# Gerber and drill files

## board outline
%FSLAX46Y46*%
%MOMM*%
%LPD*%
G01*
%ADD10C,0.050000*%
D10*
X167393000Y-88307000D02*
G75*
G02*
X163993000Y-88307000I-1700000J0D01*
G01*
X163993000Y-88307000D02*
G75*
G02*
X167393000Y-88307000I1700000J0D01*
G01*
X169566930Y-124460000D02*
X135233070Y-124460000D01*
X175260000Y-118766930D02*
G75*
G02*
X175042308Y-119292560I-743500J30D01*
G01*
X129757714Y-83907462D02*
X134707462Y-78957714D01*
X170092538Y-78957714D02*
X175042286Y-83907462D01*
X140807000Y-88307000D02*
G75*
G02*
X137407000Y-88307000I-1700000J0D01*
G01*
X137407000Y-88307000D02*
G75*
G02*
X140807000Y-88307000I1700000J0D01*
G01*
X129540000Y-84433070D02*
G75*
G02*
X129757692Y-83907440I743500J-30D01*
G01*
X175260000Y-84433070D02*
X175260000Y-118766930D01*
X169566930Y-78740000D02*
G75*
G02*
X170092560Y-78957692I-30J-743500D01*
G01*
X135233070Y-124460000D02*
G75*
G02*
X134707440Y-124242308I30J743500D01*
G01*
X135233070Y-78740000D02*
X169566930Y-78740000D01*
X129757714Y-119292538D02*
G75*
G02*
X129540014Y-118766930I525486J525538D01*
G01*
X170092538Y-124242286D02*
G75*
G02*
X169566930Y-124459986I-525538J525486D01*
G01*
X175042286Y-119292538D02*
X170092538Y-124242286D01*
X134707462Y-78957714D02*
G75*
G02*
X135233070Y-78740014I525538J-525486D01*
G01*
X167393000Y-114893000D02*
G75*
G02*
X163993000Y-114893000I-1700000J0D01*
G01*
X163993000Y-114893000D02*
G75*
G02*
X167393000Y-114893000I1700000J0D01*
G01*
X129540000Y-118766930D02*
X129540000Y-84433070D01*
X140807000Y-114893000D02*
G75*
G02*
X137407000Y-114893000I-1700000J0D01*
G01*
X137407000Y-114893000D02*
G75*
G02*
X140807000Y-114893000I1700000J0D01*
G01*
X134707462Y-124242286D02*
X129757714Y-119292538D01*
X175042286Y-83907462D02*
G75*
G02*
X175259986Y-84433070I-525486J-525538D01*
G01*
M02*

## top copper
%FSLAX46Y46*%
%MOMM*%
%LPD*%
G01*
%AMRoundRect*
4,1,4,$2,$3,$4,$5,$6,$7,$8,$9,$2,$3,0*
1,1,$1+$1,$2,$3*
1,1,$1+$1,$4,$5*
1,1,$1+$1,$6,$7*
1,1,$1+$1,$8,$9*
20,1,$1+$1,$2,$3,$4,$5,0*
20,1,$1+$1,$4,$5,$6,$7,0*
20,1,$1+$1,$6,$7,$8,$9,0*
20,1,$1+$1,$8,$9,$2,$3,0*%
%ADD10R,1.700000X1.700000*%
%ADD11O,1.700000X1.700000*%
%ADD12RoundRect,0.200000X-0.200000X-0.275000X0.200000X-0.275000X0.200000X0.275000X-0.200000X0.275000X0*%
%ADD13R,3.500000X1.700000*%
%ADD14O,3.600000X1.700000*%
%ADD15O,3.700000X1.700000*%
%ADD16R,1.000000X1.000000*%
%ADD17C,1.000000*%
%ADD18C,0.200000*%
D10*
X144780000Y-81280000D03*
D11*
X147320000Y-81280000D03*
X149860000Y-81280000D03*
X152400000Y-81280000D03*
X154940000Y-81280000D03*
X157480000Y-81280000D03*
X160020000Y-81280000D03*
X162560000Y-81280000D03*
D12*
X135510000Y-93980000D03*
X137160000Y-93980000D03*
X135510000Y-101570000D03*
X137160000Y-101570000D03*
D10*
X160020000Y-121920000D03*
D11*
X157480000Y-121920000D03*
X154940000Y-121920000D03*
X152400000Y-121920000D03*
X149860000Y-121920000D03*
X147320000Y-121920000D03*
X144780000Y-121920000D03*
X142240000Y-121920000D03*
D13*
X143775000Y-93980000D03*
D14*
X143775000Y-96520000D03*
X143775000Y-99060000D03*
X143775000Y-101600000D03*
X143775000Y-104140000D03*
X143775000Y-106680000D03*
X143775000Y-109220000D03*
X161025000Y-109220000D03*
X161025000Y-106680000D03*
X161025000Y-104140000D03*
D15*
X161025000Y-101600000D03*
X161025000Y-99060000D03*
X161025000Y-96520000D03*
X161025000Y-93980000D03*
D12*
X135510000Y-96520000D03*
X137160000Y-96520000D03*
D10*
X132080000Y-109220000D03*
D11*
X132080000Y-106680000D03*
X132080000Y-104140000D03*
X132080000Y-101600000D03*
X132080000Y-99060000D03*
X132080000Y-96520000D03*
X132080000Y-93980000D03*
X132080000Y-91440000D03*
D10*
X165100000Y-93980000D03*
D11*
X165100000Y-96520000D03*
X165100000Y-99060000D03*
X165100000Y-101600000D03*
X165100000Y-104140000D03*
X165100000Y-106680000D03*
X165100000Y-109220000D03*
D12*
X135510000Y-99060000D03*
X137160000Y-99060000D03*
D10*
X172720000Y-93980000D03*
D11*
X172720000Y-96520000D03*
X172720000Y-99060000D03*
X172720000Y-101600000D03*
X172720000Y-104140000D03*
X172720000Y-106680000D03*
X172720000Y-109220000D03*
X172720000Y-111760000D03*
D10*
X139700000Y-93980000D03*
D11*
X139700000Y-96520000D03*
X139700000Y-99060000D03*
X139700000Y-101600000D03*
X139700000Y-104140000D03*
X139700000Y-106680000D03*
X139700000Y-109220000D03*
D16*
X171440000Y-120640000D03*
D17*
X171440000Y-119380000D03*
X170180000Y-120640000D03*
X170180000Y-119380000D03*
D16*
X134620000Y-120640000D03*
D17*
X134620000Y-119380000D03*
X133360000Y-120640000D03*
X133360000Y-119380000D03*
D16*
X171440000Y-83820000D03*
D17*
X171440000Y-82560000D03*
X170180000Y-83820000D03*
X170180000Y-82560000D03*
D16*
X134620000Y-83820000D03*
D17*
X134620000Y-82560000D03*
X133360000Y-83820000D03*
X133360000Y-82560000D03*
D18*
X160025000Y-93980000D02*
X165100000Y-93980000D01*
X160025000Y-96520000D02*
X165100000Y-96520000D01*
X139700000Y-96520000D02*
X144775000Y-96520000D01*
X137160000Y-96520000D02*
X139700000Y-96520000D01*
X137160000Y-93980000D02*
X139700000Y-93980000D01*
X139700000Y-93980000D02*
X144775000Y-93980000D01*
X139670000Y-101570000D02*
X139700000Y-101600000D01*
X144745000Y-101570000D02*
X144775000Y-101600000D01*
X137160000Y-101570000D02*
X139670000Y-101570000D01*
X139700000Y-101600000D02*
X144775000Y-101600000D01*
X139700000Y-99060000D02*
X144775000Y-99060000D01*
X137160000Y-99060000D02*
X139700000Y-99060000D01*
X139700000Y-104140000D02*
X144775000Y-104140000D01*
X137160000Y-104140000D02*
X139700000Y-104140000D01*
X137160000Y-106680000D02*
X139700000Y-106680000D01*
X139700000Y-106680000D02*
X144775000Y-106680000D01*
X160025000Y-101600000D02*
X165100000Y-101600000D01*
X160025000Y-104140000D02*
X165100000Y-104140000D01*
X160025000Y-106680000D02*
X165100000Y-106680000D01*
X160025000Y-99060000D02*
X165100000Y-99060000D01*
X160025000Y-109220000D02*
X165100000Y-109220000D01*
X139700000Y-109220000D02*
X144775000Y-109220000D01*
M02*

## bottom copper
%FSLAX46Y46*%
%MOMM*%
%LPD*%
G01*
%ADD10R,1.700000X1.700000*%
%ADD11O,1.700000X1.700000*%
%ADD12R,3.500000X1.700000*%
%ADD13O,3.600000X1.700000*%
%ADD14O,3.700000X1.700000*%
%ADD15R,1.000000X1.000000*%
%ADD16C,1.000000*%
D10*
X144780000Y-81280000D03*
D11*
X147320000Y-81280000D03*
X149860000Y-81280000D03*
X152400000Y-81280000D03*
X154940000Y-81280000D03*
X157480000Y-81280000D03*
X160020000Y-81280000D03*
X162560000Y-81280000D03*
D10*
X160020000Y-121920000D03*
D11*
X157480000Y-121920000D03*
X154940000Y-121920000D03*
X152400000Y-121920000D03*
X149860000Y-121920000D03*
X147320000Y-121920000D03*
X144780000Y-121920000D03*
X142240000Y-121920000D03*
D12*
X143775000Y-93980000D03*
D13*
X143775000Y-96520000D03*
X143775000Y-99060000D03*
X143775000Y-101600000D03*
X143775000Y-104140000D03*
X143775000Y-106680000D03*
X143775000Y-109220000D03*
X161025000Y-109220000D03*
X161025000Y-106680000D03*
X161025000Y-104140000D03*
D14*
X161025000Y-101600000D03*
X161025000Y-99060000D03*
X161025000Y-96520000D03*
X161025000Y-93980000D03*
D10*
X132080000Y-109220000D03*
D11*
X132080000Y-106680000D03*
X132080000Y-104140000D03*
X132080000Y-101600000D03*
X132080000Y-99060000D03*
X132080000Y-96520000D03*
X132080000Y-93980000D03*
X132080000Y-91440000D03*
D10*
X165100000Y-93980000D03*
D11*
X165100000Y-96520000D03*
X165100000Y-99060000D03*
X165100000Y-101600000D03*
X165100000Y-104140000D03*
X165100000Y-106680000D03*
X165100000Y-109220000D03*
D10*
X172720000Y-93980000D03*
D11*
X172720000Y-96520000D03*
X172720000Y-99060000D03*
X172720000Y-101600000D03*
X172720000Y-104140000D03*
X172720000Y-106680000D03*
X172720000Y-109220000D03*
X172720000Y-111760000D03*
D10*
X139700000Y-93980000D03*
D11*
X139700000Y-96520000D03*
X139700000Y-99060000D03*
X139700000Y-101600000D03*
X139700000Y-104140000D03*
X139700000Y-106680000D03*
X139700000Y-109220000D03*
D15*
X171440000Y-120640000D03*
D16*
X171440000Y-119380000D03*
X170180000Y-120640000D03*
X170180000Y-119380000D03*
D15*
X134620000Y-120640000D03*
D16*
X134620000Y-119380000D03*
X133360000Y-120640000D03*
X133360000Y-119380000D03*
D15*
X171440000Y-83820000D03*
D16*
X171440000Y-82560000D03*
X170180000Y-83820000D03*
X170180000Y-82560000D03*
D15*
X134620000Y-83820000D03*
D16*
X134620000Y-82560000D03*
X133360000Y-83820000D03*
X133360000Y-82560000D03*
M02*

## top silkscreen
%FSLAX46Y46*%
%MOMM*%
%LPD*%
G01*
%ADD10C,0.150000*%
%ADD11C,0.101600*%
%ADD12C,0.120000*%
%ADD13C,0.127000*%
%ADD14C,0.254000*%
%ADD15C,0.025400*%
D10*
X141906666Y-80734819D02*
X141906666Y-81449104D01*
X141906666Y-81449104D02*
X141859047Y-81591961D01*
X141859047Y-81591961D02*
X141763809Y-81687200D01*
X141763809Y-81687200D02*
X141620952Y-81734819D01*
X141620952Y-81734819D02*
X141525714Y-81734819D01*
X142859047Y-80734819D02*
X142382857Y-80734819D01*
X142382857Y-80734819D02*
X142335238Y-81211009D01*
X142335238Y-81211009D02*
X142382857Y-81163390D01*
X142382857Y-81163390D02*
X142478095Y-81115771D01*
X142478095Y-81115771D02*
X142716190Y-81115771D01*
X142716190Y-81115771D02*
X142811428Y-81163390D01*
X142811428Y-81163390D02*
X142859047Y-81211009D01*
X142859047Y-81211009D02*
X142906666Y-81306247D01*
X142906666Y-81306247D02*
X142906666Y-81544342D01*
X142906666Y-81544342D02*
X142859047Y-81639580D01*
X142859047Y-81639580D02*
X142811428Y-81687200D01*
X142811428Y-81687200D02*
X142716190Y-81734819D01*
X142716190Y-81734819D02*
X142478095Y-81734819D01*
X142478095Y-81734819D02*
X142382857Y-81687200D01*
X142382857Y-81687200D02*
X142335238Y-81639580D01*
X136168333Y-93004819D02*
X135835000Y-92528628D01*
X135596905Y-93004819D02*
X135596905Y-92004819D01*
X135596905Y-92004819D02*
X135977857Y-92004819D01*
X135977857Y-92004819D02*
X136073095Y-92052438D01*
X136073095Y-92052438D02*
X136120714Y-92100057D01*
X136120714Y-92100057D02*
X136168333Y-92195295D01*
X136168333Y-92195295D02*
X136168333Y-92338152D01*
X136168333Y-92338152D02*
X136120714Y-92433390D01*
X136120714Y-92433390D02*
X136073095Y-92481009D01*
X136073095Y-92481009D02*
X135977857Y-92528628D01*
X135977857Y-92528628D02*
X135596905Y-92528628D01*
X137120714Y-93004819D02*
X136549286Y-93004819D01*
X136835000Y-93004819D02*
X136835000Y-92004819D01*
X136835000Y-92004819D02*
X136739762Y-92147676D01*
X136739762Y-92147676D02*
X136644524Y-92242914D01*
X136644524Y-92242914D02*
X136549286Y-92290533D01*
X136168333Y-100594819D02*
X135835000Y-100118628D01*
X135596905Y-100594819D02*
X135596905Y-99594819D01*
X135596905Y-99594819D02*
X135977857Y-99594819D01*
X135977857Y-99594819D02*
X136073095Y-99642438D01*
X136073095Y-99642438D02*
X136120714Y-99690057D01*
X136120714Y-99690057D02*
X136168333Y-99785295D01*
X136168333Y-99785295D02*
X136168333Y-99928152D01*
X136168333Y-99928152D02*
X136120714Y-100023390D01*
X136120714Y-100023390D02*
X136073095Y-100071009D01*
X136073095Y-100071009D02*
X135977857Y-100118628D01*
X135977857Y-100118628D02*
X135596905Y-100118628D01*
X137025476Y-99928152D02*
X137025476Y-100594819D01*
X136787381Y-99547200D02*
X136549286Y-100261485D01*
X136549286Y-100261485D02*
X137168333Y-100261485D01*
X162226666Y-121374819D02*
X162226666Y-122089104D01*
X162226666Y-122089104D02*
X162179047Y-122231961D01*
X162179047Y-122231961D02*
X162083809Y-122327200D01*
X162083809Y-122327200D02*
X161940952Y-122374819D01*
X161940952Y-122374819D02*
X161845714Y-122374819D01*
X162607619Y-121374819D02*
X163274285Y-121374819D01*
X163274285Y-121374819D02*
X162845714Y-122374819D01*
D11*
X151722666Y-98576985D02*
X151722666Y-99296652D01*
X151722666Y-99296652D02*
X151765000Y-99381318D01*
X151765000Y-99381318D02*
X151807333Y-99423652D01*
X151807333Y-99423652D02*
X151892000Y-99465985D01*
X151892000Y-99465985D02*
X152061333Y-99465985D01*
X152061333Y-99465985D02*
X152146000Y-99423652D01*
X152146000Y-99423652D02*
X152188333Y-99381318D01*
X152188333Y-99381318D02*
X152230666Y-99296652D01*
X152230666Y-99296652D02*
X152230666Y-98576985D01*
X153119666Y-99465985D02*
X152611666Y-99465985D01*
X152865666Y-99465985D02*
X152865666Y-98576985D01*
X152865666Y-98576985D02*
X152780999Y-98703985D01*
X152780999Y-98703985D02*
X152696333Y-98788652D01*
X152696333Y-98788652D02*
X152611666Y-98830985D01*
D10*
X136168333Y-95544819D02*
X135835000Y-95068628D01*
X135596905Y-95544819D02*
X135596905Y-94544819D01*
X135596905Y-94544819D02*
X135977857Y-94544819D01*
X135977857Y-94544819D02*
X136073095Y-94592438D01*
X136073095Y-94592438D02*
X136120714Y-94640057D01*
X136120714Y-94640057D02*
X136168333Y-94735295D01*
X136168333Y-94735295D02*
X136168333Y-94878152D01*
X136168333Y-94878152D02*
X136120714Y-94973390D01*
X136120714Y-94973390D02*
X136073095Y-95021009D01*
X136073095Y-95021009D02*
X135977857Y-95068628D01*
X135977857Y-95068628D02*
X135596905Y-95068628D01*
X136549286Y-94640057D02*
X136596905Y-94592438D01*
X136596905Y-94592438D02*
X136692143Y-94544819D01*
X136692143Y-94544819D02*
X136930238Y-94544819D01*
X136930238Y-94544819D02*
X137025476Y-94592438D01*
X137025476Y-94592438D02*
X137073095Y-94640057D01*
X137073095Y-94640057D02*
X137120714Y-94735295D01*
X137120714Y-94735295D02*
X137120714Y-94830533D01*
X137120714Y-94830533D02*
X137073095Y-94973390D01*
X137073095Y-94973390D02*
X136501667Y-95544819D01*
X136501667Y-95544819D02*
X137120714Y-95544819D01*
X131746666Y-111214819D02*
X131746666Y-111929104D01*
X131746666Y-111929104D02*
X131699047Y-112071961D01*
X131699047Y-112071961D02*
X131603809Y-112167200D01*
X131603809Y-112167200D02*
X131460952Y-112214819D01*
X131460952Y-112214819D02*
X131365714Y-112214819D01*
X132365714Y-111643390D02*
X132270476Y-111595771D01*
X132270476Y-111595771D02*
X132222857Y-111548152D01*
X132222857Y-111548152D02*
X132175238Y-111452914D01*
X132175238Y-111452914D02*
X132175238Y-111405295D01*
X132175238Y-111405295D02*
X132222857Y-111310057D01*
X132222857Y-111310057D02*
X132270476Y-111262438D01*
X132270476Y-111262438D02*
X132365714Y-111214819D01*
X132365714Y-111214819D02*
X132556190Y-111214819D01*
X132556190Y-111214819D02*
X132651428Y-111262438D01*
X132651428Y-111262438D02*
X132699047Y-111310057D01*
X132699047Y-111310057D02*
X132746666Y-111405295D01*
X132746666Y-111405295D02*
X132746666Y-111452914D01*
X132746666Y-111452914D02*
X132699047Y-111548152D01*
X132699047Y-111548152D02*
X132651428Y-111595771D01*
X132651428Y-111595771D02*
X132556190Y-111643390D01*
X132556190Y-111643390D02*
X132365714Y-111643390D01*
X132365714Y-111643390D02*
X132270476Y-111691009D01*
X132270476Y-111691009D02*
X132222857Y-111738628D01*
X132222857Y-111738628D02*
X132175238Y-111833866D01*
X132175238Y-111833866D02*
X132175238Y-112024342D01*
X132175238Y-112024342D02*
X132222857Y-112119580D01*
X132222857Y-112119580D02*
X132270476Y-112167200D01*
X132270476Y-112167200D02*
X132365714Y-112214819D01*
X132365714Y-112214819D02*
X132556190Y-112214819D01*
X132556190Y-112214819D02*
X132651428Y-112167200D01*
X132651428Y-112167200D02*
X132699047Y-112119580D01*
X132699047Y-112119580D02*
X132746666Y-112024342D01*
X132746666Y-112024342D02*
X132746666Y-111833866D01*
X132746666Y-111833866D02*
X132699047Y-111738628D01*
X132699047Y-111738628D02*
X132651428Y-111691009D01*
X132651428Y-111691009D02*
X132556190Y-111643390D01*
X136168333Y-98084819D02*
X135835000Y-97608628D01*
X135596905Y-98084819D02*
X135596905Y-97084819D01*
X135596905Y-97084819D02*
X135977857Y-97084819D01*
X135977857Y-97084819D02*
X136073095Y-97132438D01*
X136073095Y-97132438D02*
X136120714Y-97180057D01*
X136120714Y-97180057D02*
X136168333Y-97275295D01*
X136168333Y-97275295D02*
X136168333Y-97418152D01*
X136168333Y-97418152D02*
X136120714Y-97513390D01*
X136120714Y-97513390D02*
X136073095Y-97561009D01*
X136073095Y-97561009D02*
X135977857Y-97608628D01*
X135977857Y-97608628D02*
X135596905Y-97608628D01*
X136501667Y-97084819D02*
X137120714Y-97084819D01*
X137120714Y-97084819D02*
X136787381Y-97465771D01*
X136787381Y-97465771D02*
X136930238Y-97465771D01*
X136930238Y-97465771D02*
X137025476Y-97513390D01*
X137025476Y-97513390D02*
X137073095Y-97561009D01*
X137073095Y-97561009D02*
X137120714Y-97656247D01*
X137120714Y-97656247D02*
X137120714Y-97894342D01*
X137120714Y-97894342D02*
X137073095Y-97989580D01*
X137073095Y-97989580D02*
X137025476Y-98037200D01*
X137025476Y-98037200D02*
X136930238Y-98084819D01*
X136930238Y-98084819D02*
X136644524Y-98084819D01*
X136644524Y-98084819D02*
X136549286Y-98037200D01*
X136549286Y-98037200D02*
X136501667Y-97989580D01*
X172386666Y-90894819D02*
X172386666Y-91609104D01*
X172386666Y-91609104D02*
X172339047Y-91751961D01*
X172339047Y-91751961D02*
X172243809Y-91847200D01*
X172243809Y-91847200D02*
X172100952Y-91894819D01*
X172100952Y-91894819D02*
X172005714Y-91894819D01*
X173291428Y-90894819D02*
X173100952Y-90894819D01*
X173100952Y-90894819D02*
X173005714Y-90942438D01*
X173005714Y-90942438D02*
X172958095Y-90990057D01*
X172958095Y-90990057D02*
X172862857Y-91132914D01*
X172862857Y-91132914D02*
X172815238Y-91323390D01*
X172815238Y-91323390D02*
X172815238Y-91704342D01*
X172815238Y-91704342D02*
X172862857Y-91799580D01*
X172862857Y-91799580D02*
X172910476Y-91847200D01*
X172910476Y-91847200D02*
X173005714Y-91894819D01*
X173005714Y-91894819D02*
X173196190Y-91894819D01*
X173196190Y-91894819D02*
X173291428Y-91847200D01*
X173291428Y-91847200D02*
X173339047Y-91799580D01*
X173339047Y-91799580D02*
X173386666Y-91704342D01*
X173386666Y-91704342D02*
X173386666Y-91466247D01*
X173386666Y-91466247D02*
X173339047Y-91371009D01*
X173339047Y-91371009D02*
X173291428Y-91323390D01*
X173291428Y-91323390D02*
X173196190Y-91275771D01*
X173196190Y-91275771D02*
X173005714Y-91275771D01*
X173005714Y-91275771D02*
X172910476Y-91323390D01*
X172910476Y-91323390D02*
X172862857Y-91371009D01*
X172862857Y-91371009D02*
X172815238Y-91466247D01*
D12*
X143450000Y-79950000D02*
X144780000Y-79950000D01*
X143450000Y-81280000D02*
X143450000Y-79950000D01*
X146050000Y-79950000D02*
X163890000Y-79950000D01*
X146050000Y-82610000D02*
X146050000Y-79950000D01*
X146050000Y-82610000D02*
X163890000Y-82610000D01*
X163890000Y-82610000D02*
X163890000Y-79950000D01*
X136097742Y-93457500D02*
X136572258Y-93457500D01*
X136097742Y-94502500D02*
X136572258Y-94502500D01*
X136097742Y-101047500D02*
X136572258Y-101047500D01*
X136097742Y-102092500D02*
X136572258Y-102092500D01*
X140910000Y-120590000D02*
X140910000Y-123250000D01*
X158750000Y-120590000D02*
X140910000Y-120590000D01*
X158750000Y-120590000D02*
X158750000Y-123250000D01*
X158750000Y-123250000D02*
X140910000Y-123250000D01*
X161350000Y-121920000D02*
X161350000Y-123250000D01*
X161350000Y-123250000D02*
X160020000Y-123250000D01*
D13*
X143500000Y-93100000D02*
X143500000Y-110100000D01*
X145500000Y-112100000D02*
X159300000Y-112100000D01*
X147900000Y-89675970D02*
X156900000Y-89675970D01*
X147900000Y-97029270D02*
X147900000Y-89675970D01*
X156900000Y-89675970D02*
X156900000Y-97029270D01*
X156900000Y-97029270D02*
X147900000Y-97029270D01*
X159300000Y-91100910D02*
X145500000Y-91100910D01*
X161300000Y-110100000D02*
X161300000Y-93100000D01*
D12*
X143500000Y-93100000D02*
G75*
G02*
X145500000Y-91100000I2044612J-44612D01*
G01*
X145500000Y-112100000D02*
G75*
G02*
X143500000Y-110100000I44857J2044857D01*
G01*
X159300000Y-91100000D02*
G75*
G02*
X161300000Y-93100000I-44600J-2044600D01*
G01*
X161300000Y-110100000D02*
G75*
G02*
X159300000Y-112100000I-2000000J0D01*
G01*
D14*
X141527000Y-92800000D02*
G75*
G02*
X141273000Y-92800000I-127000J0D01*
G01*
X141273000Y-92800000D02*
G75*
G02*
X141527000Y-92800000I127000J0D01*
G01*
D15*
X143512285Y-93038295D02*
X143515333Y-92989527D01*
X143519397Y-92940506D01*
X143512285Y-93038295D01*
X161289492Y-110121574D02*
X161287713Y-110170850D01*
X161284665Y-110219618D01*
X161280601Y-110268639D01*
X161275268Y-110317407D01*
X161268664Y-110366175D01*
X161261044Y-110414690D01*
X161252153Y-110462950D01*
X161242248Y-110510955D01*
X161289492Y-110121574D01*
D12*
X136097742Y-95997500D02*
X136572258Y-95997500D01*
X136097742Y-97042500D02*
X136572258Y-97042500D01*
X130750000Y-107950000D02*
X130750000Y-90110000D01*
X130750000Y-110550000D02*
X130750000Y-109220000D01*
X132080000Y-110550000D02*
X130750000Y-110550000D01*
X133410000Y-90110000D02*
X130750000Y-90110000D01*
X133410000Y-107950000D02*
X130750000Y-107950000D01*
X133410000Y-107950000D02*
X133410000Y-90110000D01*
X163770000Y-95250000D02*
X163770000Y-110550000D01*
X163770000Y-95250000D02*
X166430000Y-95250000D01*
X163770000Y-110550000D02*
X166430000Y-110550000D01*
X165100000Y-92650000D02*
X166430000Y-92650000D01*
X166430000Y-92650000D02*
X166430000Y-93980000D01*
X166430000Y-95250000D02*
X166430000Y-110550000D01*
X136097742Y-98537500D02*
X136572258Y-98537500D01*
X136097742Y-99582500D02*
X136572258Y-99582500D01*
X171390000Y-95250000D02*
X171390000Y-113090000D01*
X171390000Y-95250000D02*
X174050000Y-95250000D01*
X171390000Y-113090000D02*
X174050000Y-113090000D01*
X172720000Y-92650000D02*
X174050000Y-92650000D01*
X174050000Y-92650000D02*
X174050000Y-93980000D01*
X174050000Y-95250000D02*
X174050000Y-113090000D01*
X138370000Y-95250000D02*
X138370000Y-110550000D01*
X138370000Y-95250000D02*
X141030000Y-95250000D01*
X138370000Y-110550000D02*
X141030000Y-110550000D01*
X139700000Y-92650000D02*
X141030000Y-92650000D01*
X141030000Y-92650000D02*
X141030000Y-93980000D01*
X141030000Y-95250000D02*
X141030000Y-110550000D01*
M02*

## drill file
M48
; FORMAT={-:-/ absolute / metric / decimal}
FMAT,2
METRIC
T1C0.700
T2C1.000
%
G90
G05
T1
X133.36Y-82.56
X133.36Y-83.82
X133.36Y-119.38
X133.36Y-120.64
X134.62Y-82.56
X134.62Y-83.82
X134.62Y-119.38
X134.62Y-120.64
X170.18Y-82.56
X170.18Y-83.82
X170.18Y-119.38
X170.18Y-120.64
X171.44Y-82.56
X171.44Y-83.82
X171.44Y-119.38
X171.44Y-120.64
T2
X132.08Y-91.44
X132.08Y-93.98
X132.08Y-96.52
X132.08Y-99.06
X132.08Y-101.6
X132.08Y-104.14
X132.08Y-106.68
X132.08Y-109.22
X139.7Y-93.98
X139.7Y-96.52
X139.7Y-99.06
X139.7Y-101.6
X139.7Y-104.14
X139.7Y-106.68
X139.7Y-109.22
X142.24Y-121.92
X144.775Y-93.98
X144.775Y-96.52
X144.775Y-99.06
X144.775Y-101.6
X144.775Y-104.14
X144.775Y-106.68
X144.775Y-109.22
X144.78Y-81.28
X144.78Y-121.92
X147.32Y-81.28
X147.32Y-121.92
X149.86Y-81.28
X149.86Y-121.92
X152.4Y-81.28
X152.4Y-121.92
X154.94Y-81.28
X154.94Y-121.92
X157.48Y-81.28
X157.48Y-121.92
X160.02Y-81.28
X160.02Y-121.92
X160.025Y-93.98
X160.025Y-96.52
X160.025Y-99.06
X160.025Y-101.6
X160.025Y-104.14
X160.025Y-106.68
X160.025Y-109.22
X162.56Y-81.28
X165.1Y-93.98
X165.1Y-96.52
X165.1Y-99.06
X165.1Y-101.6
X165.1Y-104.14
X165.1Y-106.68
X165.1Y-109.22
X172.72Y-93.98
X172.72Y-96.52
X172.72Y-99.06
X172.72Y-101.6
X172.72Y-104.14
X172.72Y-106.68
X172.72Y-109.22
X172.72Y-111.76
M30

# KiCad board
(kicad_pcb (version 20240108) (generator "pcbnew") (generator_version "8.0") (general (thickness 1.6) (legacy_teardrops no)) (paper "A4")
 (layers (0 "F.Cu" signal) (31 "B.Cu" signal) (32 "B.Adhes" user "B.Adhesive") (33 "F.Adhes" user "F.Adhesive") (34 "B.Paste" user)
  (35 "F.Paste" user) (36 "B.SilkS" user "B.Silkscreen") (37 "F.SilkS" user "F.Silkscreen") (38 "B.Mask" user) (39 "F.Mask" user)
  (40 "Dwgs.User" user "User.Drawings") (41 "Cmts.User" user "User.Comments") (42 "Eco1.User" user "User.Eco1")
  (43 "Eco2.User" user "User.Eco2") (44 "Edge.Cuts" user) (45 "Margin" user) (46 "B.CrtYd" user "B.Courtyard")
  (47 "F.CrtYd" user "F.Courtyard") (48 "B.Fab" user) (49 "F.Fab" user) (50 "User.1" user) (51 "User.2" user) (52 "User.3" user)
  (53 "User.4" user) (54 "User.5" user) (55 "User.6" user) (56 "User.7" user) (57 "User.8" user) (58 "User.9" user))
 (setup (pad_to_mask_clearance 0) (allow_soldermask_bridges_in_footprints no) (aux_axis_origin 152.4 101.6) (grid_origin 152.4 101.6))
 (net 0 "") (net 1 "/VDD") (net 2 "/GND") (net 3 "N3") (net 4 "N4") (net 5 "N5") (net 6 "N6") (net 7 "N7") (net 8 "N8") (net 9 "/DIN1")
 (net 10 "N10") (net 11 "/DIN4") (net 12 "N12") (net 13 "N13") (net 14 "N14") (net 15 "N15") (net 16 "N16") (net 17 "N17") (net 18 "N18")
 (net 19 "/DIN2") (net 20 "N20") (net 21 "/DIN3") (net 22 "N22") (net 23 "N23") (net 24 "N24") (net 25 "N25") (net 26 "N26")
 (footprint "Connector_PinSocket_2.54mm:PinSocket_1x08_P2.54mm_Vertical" (layer "F.Cu") (at 144.78 81.28 90)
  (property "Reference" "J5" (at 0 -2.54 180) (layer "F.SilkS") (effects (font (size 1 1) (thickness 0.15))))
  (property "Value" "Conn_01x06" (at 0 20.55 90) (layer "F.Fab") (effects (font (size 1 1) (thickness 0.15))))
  (fp_line (start 1.33 -1.33) (end 1.33 0) (stroke (width 0.12) (type solid)) (layer "F.SilkS"))
  (fp_line (start 0 -1.33) (end 1.33 -1.33) (stroke (width 0.12) (type solid)) (layer "F.SilkS"))
  (fp_line (start 1.33 1.27) (end 1.33 19.11) (stroke (width 0.12) (type solid)) (layer "F.SilkS"))
  (fp_line (start -1.33 1.27) (end 1.33 1.27) (stroke (width 0.12) (type solid)) (layer "F.SilkS"))
  (fp_line (start -1.33 1.27) (end -1.33 19.11) (stroke (width 0.12) (type solid)) (layer "F.SilkS"))
  (fp_line (start -1.33 19.11) (end 1.33 19.11) (stroke (width 0.12) (type solid)) (layer "F.SilkS"))
  (pad "1" thru_hole rect (at 0 0 90) (size 1.7 1.7) (drill 1) (layers "*.Cu" "*.Mask") (remove_unused_layers no) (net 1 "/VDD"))
  (pad "2" thru_hole oval (at 0 2.54 90) (size 1.7 1.7) (drill 1) (layers "*.Cu" "*.Mask") (remove_unused_layers no) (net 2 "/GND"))
  (pad "3" thru_hole oval (at 0 5.08 90) (size 1.7 1.7) (drill 1) (layers "*.Cu" "*.Mask") (remove_unused_layers no) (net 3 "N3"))
  (pad "4" thru_hole oval (at 0 7.62 90) (size 1.7 1.7) (drill 1) (layers "*.Cu" "*.Mask") (remove_unused_layers no) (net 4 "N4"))
  (pad "5" thru_hole oval (at 0 10.16 90) (size 1.7 1.7) (drill 1) (layers "*.Cu" "*.Mask") (remove_unused_layers no) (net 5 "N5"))
  (pad "6" thru_hole oval (at 0 12.7 90) (size 1.7 1.7) (drill 1) (layers "*.Cu" "*.Mask") (remove_unused_layers no) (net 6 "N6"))
  (pad "7" thru_hole oval (at 0 15.24 90) (size 1.7 1.7) (drill 1) (layers "*.Cu" "*.Mask") (remove_unused_layers no) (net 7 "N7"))
  (pad "8" thru_hole oval (at 0 17.78 90) (size 1.7 1.7) (drill 1) (layers "*.Cu" "*.Mask") (remove_unused_layers no) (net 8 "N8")))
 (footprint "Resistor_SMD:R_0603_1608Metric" (layer "F.Cu") (at 136.335 93.98)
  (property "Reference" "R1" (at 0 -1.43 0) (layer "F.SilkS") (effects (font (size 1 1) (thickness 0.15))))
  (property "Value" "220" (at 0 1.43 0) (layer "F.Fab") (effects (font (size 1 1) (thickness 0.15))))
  (fp_line (start -0.237258 -0.5225) (end 0.237258 -0.5225) (stroke (width 0.12) (type solid)) (layer "F.SilkS"))
  (fp_line (start -0.237258 0.5225) (end 0.237258 0.5225) (stroke (width 0.12) (type solid)) (layer "F.SilkS"))
  (pad "1" smd roundrect (at -0.825 0) (size 0.8 0.95) (layers "F.Cu" "F.Paste" "F.Mask") (roundrect_rratio 0.25) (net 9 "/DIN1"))
  (pad "2" smd roundrect (at 0.825 0) (size 0.8 0.95) (layers "F.Cu" "F.Paste" "F.Mask") (roundrect_rratio 0.25) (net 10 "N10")))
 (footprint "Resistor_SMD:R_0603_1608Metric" (layer "F.Cu") (at 136.335 101.57)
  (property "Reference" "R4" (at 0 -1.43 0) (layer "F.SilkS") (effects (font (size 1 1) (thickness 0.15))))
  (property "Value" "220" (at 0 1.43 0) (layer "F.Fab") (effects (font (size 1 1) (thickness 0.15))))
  (fp_line (start -0.237258 -0.5225) (end 0.237258 -0.5225) (stroke (width 0.12) (type solid)) (layer "F.SilkS"))
  (fp_line (start -0.237258 0.5225) (end 0.237258 0.5225) (stroke (width 0.12) (type solid)) (layer "F.SilkS"))
  (pad "1" smd roundrect (at -0.825 0) (size 0.8 0.95) (layers "F.Cu" "F.Paste" "F.Mask") (roundrect_rratio 0.25) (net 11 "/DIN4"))
  (pad "2" smd roundrect (at 0.825 0) (size 0.8 0.95) (layers "F.Cu" "F.Paste" "F.Mask") (roundrect_rratio 0.25) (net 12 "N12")))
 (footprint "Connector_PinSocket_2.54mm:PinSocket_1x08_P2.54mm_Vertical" (layer "F.Cu") (at 160.02 121.92 -90)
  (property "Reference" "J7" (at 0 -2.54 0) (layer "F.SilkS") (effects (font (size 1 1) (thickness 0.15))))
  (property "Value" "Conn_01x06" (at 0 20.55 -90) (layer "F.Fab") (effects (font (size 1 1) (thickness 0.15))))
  (fp_line (start -1.33 19.11) (end 1.33 19.11) (stroke (width 0.12) (type solid)) (layer "F.SilkS"))
  (fp_line (start -1.33 1.27) (end -1.33 19.11) (stroke (width 0.12) (type solid)) (layer "F.SilkS"))
  (fp_line (start -1.33 1.27) (end 1.33 1.27) (stroke (width 0.12) (type solid)) (layer "F.SilkS"))
  (fp_line (start 1.33 1.27) (end 1.33 19.11) (stroke (width 0.12) (type solid)) (layer "F.SilkS"))
  (fp_line (start 0 -1.33) (end 1.33 -1.33) (stroke (width 0.12) (type solid)) (layer "F.SilkS"))
  (fp_line (start 1.33 -1.33) (end 1.33 0) (stroke (width 0.12) (type solid)) (layer "F.SilkS"))
  (pad "1" thru_hole rect (at 0 0 270) (size 1.7 1.7) (drill 1) (layers "*.Cu" "*.Mask") (remove_unused_layers no) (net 1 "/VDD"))
  (pad "2" thru_hole oval (at 0 2.54 270) (size 1.7 1.7) (drill 1) (layers "*.Cu" "*.Mask") (remove_unused_layers no) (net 2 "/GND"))
  (pad "3" thru_hole oval (at 0 5.08 270) (size 1.7 1.7) (drill 1) (layers "*.Cu" "*.Mask") (remove_unused_layers no) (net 3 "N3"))
  (pad "4" thru_hole oval (at 0 7.62 270) (size 1.7 1.7) (drill 1) (layers "*.Cu" "*.Mask") (remove_unused_layers no) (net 4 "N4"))
  (pad "5" thru_hole oval (at 0 10.16 270) (size 1.7 1.7) (drill 1) (layers "*.Cu" "*.Mask") (remove_unused_layers no) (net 5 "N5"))
  (pad "6" thru_hole oval (at 0 12.7 270) (size 1.7 1.7) (drill 1) (layers "*.Cu" "*.Mask") (remove_unused_layers no) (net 6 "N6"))
  (pad "7" thru_hole oval (at 0 15.24 270) (size 1.7 1.7) (drill 1) (layers "*.Cu" "*.Mask") (remove_unused_layers no) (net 7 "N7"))
  (pad "8" thru_hole oval (at 0 17.78 270) (size 1.7 1.7) (drill 1) (layers "*.Cu" "*.Mask") (remove_unused_layers no) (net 8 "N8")))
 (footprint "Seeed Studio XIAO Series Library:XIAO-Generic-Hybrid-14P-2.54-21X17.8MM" (layer "F.Cu") (at 152.4 101.6)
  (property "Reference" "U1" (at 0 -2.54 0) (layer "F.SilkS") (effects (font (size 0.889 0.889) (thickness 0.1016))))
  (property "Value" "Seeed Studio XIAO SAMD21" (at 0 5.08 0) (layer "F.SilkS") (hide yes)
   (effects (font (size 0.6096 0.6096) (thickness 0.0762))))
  (fp_line (start -8.9 -8.5) (end -8.9 8.5) (stroke (width 0.127) (type solid)) (layer "F.SilkS"))
  (fp_line (start -6.9 10.5) (end 6.9 10.5) (stroke (width 0.127) (type solid)) (layer "F.SilkS"))
  (fp_line (start -4.5 -11.92403) (end 4.5 -11.92403) (stroke (width 0.127) (type solid)) (layer "F.SilkS"))
  (fp_line (start -4.5 -4.57073) (end -4.5 -11.92403) (stroke (width 0.127) (type solid)) (layer "F.SilkS"))
  (fp_line (start 4.5 -11.92403) (end 4.5 -4.57073) (stroke (width 0.127) (type solid)) (layer "F.SilkS"))
  (fp_line (start 4.5 -4.57073) (end -4.5 -4.57073) (stroke (width 0.127) (type solid)) (layer "F.SilkS"))
  (fp_line (start 6.9 -10.49909) (end -6.9 -10.49909) (stroke (width 0.127) (type solid)) (layer "F.SilkS"))
  (fp_line (start 8.9 8.5) (end 8.9 -8.5) (stroke (width 0.127) (type solid)) (layer "F.SilkS"))
  (fp_arc (start -8.9 -8.5) (mid -8.301491 -9.901491) (end -6.9 -10.5) (stroke (width 0.12) (type solid)) (layer "F.SilkS"))
  (fp_arc (start -6.9 10.5) (mid -8.301423 9.901423) (end -8.9 8.5) (stroke (width 0.12) (type solid)) (layer "F.SilkS"))
  (fp_arc (start 6.9 -10.5) (mid 8.301492 -9.901492) (end 8.9 -8.5) (stroke (width 0.12) (type solid)) (layer "F.SilkS"))
  (fp_arc (start 8.9 8.5) (mid 8.314214 9.914214) (end 6.9 10.5) (stroke (width 0.12) (type solid)) (layer "F.SilkS"))
  (fp_circle (center -11 -8.8) (end -11 -9.054) (stroke (width 0) (type solid)) (fill solid) (layer "F.SilkS"))
  (fp_poly
   (pts (xy -8.887715 -8.561705) (xy -8.884667 -8.610473) (xy -8.880603 -8.659494)) (stroke (width 0.0254) (type solid)) (fill none)
   (layer "F.SilkS"))
  (fp_poly
   (pts (xy 8.889492 8.521574) (xy 8.887713 8.57085) (xy 8.884665 8.619618) (xy 8.880601 8.668639) (xy 8.875268 8.717407)
    (xy 8.868664 8.766175) (xy 8.861044 8.81469) (xy 8.852153 8.86295) (xy 8.842248 8.910955))
   (stroke (width 0.0254) (type solid)) (fill none) (layer "F.SilkS"))
  (pad "1" thru_hole rect (at -7.625 -7.62) (size 3.5 1.7) (drill 1 (offset -1 0)) (layers "*.Cu" "*.Mask") (remove_unused_layers no)
   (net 3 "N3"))
  (pad "2" thru_hole oval (at -7.625 -5.08) (size 3.6 1.7) (drill 1 (offset -1 0)) (layers "*.Cu" "*.Mask") (remove_unused_layers no)
   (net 4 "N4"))
  (pad "3" thru_hole oval (at -7.625 -2.54) (size 3.6 1.7) (drill 1 (offset -1 0)) (layers "*.Cu" "*.Mask") (remove_unused_layers no)
   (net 5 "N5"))
  (pad "4" thru_hole oval (at -7.625 0) (size 3.6 1.7) (drill 1 (offset -1 0)) (layers "*.Cu" "*.Mask") (remove_unused_layers no)
   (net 6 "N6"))
  (pad "5" thru_hole oval (at -7.625 2.54) (size 3.6 1.7) (drill 1 (offset -1 0)) (layers "*.Cu" "*.Mask") (remove_unused_layers no)
   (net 7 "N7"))
  (pad "6" thru_hole oval (at -7.625 5.08 180) (size 3.6 1.7) (drill 1 (offset 1 0)) (layers "*.Cu" "*.Mask") (remove_unused_layers no)
   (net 8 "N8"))
  (pad "7" thru_hole oval (at -7.625 7.62) (size 3.6 1.7) (drill 1 (offset -1 0)) (layers "*.Cu" "*.Mask") (remove_unused_layers no)
   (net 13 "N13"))
  (pad "8" thru_hole oval (at 7.625 7.62) (size 3.6 1.7) (drill 1 (offset 1 0)) (layers "*.Cu" "*.Mask") (remove_unused_layers no)
   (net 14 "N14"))
  (pad "9" thru_hole oval (at 7.625 5.08) (size 3.6 1.7) (drill 1 (offset 1 0)) (layers "*.Cu" "*.Mask") (remove_unused_layers no)
   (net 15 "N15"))
  (pad "10" thru_hole oval (at 7.625 2.54) (size 3.6 1.7) (drill 1 (offset 1 0)) (layers "*.Cu" "*.Mask") (remove_unused_layers no)
   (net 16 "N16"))
  (pad "11" thru_hole oval (at 7.625 0) (size 3.7 1.7) (drill 1 (offset 1 0)) (layers "*.Cu" "*.Mask") (remove_unused_layers no)
   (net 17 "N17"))
  (pad "12" thru_hole oval (at 7.625 -2.54) (size 3.7 1.7) (drill 1 (offset 1 0)) (layers "*.Cu" "*.Mask") (remove_unused_layers no)
   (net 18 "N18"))
  (pad "13" thru_hole oval (at 7.625 -5.08) (size 3.7 1.7) (drill 1 (offset 1 0)) (layers "*.Cu" "*.Mask") (remove_unused_layers no)
   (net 1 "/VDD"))
  (pad "14" thru_hole oval (at 7.625 -7.62) (size 3.7 1.7) (drill 1 (offset 1 0)) (layers "*.Cu" "*.Mask") (remove_unused_layers no)
   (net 2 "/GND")))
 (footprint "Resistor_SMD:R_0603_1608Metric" (layer "F.Cu") (at 136.335 96.52)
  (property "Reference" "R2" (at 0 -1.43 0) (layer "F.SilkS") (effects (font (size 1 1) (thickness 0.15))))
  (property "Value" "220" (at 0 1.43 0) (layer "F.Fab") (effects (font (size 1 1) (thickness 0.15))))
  (fp_line (start -0.237258 -0.5225) (end 0.237258 -0.5225) (stroke (width 0.12) (type solid)) (layer "F.SilkS"))
  (fp_line (start -0.237258 0.5225) (end 0.237258 0.5225) (stroke (width 0.12) (type solid)) (layer "F.SilkS"))
  (pad "1" smd roundrect (at -0.825 0) (size 0.8 0.95) (layers "F.Cu" "F.Paste" "F.Mask") (roundrect_rratio 0.25) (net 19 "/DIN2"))
  (pad "2" smd roundrect (at 0.825 0) (size 0.8 0.95) (layers "F.Cu" "F.Paste" "F.Mask") (roundrect_rratio 0.25) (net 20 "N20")))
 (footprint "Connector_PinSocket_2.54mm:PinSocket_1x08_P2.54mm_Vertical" (layer "F.Cu") (at 132.08 109.22 180)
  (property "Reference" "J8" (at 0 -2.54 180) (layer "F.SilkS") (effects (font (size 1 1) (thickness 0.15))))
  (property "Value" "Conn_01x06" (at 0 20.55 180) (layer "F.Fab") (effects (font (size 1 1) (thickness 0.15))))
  (fp_line (start 1.33 1.27) (end 1.33 19.11) (stroke (width 0.12) (type solid)) (layer "F.SilkS"))
  (fp_line (start 1.33 -1.33) (end 1.33 0) (stroke (width 0.12) (type solid)) (layer "F.SilkS"))
  (fp_line (start 0 -1.33) (end 1.33 -1.33) (stroke (width 0.12) (type solid)) (layer "F.SilkS"))
  (fp_line (start -1.33 19.11) (end 1.33 19.11) (stroke (width 0.12) (type solid)) (layer "F.SilkS"))
  (fp_line (start -1.33 1.27) (end 1.33 1.27) (stroke (width 0.12) (type solid)) (layer "F.SilkS"))
  (fp_line (start -1.33 1.27) (end -1.33 19.11) (stroke (width 0.12) (type solid)) (layer "F.SilkS"))
  (pad "1" thru_hole rect (at 0 0 180) (size 1.7 1.7) (drill 1) (layers "*.Cu" "*.Mask") (remove_unused_layers no) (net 1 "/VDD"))
  (pad "2" thru_hole oval (at 0 2.54 180) (size 1.7 1.7) (drill 1) (layers "*.Cu" "*.Mask") (remove_unused_layers no) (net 2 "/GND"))
  (pad "3" thru_hole oval (at 0 5.08 180) (size 1.7 1.7) (drill 1) (layers "*.Cu" "*.Mask") (remove_unused_layers no) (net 3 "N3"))
  (pad "4" thru_hole oval (at 0 7.62 180) (size 1.7 1.7) (drill 1) (layers "*.Cu" "*.Mask") (remove_unused_layers no) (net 4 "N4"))
  (pad "5" thru_hole oval (at 0 10.16 180) (size 1.7 1.7) (drill 1) (layers "*.Cu" "*.Mask") (remove_unused_layers no) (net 5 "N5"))
  (pad "6" thru_hole oval (at 0 12.7 180) (size 1.7 1.7) (drill 1) (layers "*.Cu" "*.Mask") (remove_unused_layers no) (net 6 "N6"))
  (pad "7" thru_hole oval (at 0 15.24 180) (size 1.7 1.7) (drill 1) (layers "*.Cu" "*.Mask") (remove_unused_layers no) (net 7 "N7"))
  (pad "8" thru_hole oval (at 0 17.78 180) (size 1.7 1.7) (drill 1) (layers "*.Cu" "*.Mask") (remove_unused_layers no) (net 8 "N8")))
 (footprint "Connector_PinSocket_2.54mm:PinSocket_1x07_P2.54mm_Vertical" (layer "F.Cu") (at 165.1 93.98)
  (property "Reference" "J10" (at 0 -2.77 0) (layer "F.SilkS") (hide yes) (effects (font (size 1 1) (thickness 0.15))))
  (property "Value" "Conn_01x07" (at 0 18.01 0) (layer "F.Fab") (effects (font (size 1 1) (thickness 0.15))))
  (fp_line (start -1.33 1.27) (end -1.33 16.57) (stroke (width 0.12) (type solid)) (layer "F.SilkS"))
  (fp_line (start -1.33 1.27) (end 1.33 1.27) (stroke (width 0.12) (type solid)) (layer "F.SilkS"))
  (fp_line (start -1.33 16.57) (end 1.33 16.57) (stroke (width 0.12) (type solid)) (layer "F.SilkS"))
  (fp_line (start 0 -1.33) (end 1.33 -1.33) (stroke (width 0.12) (type solid)) (layer "F.SilkS"))
  (fp_line (start 1.33 -1.33) (end 1.33 0) (stroke (width 0.12) (type solid)) (layer "F.SilkS"))
  (fp_line (start 1.33 1.27) (end 1.33 16.57) (stroke (width 0.12) (type solid)) (layer "F.SilkS"))
  (pad "1" thru_hole rect (at 0 0) (size 1.7 1.7) (drill 1) (layers "*.Cu" "*.Mask") (remove_unused_layers no) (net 2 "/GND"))
  (pad "2" thru_hole oval (at 0 2.54) (size 1.7 1.7) (drill 1) (layers "*.Cu" "*.Mask") (remove_unused_layers no) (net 1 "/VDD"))
  (pad "3" thru_hole oval (at 0 5.08) (size 1.7 1.7) (drill 1) (layers "*.Cu" "*.Mask") (remove_unused_layers no) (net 18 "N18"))
  (pad "4" thru_hole oval (at 0 7.62) (size 1.7 1.7) (drill 1) (layers "*.Cu" "*.Mask") (remove_unused_layers no) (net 17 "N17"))
  (pad "5" thru_hole oval (at 0 10.16) (size 1.7 1.7) (drill 1) (layers "*.Cu" "*.Mask") (remove_unused_layers no) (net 16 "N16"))
  (pad "6" thru_hole oval (at 0 12.7) (size 1.7 1.7) (drill 1) (layers "*.Cu" "*.Mask") (remove_unused_layers no) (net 15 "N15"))
  (pad "7" thru_hole oval (at 0 15.24) (size 1.7 1.7) (drill 1) (layers "*.Cu" "*.Mask") (remove_unused_layers no) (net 14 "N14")))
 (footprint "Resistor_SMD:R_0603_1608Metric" (layer "F.Cu") (at 136.335 99.06)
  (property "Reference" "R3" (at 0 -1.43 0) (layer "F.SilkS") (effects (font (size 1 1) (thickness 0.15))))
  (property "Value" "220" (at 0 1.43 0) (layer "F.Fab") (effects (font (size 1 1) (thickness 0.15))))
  (fp_line (start -0.237258 -0.5225) (end 0.237258 -0.5225) (stroke (width 0.12) (type solid)) (layer "F.SilkS"))
  (fp_line (start -0.237258 0.5225) (end 0.237258 0.5225) (stroke (width 0.12) (type solid)) (layer "F.SilkS"))
  (pad "1" smd roundrect (at -0.825 0) (size 0.8 0.95) (layers "F.Cu" "F.Paste" "F.Mask") (roundrect_rratio 0.25) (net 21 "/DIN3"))
  (pad "2" smd roundrect (at 0.825 0) (size 0.8 0.95) (layers "F.Cu" "F.Paste" "F.Mask") (roundrect_rratio 0.25) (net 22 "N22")))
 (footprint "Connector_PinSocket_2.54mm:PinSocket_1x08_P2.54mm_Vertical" (layer "F.Cu") (at 172.72 93.98)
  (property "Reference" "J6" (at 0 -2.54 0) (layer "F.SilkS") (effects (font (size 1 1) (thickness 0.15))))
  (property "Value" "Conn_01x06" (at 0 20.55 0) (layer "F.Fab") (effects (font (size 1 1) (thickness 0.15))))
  (fp_line (start -1.33 1.27) (end -1.33 19.11) (stroke (width 0.12) (type solid)) (layer "F.SilkS"))
  (fp_line (start -1.33 1.27) (end 1.33 1.27) (stroke (width 0.12) (type solid)) (layer "F.SilkS"))
  (fp_line (start -1.33 19.11) (end 1.33 19.11) (stroke (width 0.12) (type solid)) (layer "F.SilkS"))
  (fp_line (start 0 -1.33) (end 1.33 -1.33) (stroke (width 0.12) (type solid)) (layer "F.SilkS"))
  (fp_line (start 1.33 -1.33) (end 1.33 0) (stroke (width 0.12) (type solid)) (layer "F.SilkS"))
  (fp_line (start 1.33 1.27) (end 1.33 19.11) (stroke (width 0.12) (type solid)) (layer "F.SilkS"))
  (pad "1" thru_hole rect (at 0 0) (size 1.7 1.7) (drill 1) (layers "*.Cu" "*.Mask") (remove_unused_layers no) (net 1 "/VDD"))
  (pad "2" thru_hole oval (at 0 2.54) (size 1.7 1.7) (drill 1) (layers "*.Cu" "*.Mask") (remove_unused_layers no) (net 2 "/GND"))
  (pad "3" thru_hole oval (at 0 5.08) (size 1.7 1.7) (drill 1) (layers "*.Cu" "*.Mask") (remove_unused_layers no) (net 3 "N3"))
  (pad "4" thru_hole oval (at 0 7.62) (size 1.7 1.7) (drill 1) (layers "*.Cu" "*.Mask") (remove_unused_layers no) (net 4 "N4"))
  (pad "5" thru_hole oval (at 0 10.16) (size 1.7 1.7) (drill 1) (layers "*.Cu" "*.Mask") (remove_unused_layers no) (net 5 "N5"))
  (pad "6" thru_hole oval (at 0 12.7) (size 1.7 1.7) (drill 1) (layers "*.Cu" "*.Mask") (remove_unused_layers no) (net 6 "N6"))
  (pad "7" thru_hole oval (at 0 15.24) (size 1.7 1.7) (drill 1) (layers "*.Cu" "*.Mask") (remove_unused_layers no) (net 7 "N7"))
  (pad "8" thru_hole oval (at 0 17.78) (size 1.7 1.7) (drill 1) (layers "*.Cu" "*.Mask") (remove_unused_layers no) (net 8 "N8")))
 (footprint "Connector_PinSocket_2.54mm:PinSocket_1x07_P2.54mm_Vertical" (layer "F.Cu") (at 139.7 93.98)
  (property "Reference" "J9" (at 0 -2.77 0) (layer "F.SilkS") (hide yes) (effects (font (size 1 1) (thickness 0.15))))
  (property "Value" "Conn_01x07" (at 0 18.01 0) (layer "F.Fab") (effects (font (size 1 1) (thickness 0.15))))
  (fp_line (start -1.33 1.27) (end -1.33 16.57) (stroke (width 0.12) (type solid)) (layer "F.SilkS"))
  (fp_line (start -1.33 1.27) (end 1.33 1.27) (stroke (width 0.12) (type solid)) (layer "F.SilkS"))
  (fp_line (start -1.33 16.57) (end 1.33 16.57) (stroke (width 0.12) (type solid)) (layer "F.SilkS"))
  (fp_line (start 0 -1.33) (end 1.33 -1.33) (stroke (width 0.12) (type solid)) (layer "F.SilkS"))
  (fp_line (start 1.33 -1.33) (end 1.33 0) (stroke (width 0.12) (type solid)) (layer "F.SilkS"))
  (fp_line (start 1.33 1.27) (end 1.33 16.57) (stroke (width 0.12) (type solid)) (layer "F.SilkS"))
  (pad "1" thru_hole rect (at 0 0) (size 1.7 1.7) (drill 1) (layers "*.Cu" "*.Mask") (remove_unused_layers no) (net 3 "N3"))
  (pad "2" thru_hole oval (at 0 2.54) (size 1.7 1.7) (drill 1) (layers "*.Cu" "*.Mask") (remove_unused_layers no) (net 4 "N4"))
  (pad "3" thru_hole oval (at 0 5.08) (size 1.7 1.7) (drill 1) (layers "*.Cu" "*.Mask") (remove_unused_layers no) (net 5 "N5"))
  (pad "4" thru_hole oval (at 0 7.62) (size 1.7 1.7) (drill 1) (layers "*.Cu" "*.Mask") (remove_unused_layers no) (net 6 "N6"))
  (pad "5" thru_hole oval (at 0 10.16) (size 1.7 1.7) (drill 1) (layers "*.Cu" "*.Mask") (remove_unused_layers no) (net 7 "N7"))
  (pad "6" thru_hole oval (at 0 12.7) (size 1.7 1.7) (drill 1) (layers "*.Cu" "*.Mask") (remove_unused_layers no) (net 8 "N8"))
  (pad "7" thru_hole oval (at 0 15.24) (size 1.7 1.7) (drill 1) (layers "*.Cu" "*.Mask") (remove_unused_layers no) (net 13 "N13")))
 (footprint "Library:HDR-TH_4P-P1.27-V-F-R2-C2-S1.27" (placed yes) (layer "B.Cu") (at 170.81 120.01 180)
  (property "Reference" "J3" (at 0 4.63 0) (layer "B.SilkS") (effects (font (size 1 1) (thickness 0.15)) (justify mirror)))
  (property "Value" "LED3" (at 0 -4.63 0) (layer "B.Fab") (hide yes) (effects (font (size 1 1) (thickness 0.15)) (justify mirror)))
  (pad "1" thru_hole rect (at -0.63 -0.63 180) (size 1 1) (drill 0.700024) (layers "*.Cu" "*.Mask") (remove_unused_layers no)
   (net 21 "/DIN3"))
  (pad "2" thru_hole circle (at -0.63 0.63 180) (size 1 1) (drill 0.700024) (layers "*.Cu" "*.Mask") (remove_unused_layers no)
   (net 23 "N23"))
  (pad "3" thru_hole circle (at 0.63 -0.63 180) (size 1 1) (drill 0.700024) (layers "*.Cu" "*.Mask") (remove_unused_layers no)
   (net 1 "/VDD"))
  (pad "4" thru_hole circle (at 0.63 0.63 180) (size 1 1) (drill 0.700024) (layers "*.Cu" "*.Mask") (remove_unused_layers no) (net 2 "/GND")))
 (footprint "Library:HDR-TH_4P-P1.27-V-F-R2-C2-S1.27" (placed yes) (layer "B.Cu") (at 133.99 120.01 180)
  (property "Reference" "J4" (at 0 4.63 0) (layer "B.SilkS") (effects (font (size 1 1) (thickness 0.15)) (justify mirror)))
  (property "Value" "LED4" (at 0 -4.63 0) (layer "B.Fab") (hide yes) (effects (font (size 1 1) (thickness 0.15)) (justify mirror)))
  (pad "1" thru_hole rect (at -0.63 -0.63 180) (size 1 1) (drill 0.700024) (layers "*.Cu" "*.Mask") (remove_unused_layers no)
   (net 11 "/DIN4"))
  (pad "2" thru_hole circle (at -0.63 0.63 180) (size 1 1) (drill 0.700024) (layers "*.Cu" "*.Mask") (remove_unused_layers no)
   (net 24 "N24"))
  (pad "3" thru_hole circle (at 0.63 -0.63 180) (size 1 1) (drill 0.700024) (layers "*.Cu" "*.Mask") (remove_unused_layers no)
   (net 1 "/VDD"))
  (pad "4" thru_hole circle (at 0.63 0.63 180) (size 1 1) (drill 0.700024) (layers "*.Cu" "*.Mask") (remove_unused_layers no) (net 2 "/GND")))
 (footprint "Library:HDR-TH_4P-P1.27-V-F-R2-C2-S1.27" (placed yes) (layer "B.Cu") (at 170.81 83.19 180)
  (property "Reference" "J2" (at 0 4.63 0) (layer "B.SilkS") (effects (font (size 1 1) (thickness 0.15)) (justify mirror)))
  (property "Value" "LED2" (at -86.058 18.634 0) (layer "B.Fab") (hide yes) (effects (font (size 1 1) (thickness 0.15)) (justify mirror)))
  (pad "1" thru_hole rect (at -0.63 -0.63 180) (size 1 1) (drill 0.700024) (layers "*.Cu" "*.Mask") (remove_unused_layers no)
   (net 19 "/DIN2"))
  (pad "2" thru_hole circle (at -0.63 0.63 180) (size 1 1) (drill 0.700024) (layers "*.Cu" "*.Mask") (remove_unused_layers no)
   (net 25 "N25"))
  (pad "3" thru_hole circle (at 0.63 -0.63 180) (size 1 1) (drill 0.700024) (layers "*.Cu" "*.Mask") (remove_unused_layers no)
   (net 1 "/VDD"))
  (pad "4" thru_hole circle (at 0.63 0.63 180) (size 1 1) (drill 0.700024) (layers "*.Cu" "*.Mask") (remove_unused_layers no) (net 2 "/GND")))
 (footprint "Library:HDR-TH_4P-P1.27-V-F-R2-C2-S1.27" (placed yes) (layer "B.Cu") (at 133.99 83.19 180)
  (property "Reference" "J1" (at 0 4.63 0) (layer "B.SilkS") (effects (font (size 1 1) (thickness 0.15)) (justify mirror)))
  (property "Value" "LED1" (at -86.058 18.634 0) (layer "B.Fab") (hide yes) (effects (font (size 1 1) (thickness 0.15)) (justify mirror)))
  (pad "1" thru_hole rect (at -0.63 -0.63 180) (size 1 1) (drill 0.700024) (layers "*.Cu" "*.Mask") (remove_unused_layers no)
   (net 9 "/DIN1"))
  (pad "2" thru_hole circle (at -0.63 0.63 180) (size 1 1) (drill 0.700024) (layers "*.Cu" "*.Mask") (remove_unused_layers no)
   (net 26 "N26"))
  (pad "3" thru_hole circle (at 0.63 -0.63 180) (size 1 1) (drill 0.700024) (layers "*.Cu" "*.Mask") (remove_unused_layers no)
   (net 1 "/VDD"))
  (pad "4" thru_hole circle (at 0.63 0.63 180) (size 1 1) (drill 0.700024) (layers "*.Cu" "*.Mask") (remove_unused_layers no) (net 2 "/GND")))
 (gr_circle (center 165.693 88.307) (end 167.393 88.307) (stroke (width 0.05) (type default)) (fill none) (layer "Edge.Cuts"))
 (gr_line (start 169.56693 124.46) (end 135.23307 124.46) (stroke (width 0.05) (type default)) (layer "Edge.Cuts"))
 (gr_arc (start 175.26 118.76693) (mid 175.203407 119.051379) (end 175.042286 119.292538) (stroke (width 0.05) (type default))
  (layer "Edge.Cuts"))
 (gr_line (start 129.757714 83.907462) (end 134.707462 78.957714) (stroke (width 0.05) (type default)) (layer "Edge.Cuts"))
 (gr_line (start 170.092538 78.957714) (end 175.042286 83.907462) (stroke (width 0.05) (type default)) (layer "Edge.Cuts"))
 (gr_circle (center 139.107 88.307) (end 140.807 88.307) (stroke (width 0.05) (type default)) (fill none) (layer "Edge.Cuts"))
 (gr_arc (start 129.54 84.43307) (mid 129.596593 84.148621) (end 129.757714 83.907462) (stroke (width 0.05) (type default))
  (layer "Edge.Cuts"))
 (gr_line (start 175.26 84.43307) (end 175.26 118.76693) (stroke (width 0.05) (type default)) (layer "Edge.Cuts"))
 (gr_arc (start 169.56693 78.74) (mid 169.851379 78.796593) (end 170.092538 78.957714) (stroke (width 0.05) (type default))
  (layer "Edge.Cuts"))
 (gr_arc (start 135.23307 124.46) (mid 134.948621 124.403407) (end 134.707462 124.242286) (stroke (width 0.05) (type default))
  (layer "Edge.Cuts"))
 (gr_line (start 135.23307 78.74) (end 169.56693 78.74) (stroke (width 0.05) (type default)) (layer "Edge.Cuts"))
 (gr_arc (start 129.757714 119.292538) (mid 129.596568 119.05139) (end 129.54 118.76693) (stroke (width 0.05) (type default))
  (layer "Edge.Cuts"))
 (gr_arc (start 170.092538 124.242286) (mid 169.85139 124.403432) (end 169.56693 124.46) (stroke (width 0.05) (type default))
  (layer "Edge.Cuts"))
 (gr_line (start 175.042286 119.292538) (end 170.092538 124.242286) (stroke (width 0.05) (type default)) (layer "Edge.Cuts"))
 (gr_arc (start 134.707462 78.957714) (mid 134.94861 78.796568) (end 135.23307 78.74) (stroke (width 0.05) (type default))
  (layer "Edge.Cuts"))
 (gr_circle (center 165.693 114.893) (end 167.393 114.893) (stroke (width 0.05) (type default)) (fill none) (layer "Edge.Cuts"))
 (gr_line (start 129.54 118.76693) (end 129.54 84.43307) (stroke (width 0.05) (type default)) (layer "Edge.Cuts"))
 (gr_circle (center 139.107 114.893) (end 140.807 114.893) (stroke (width 0.05) (type default)) (fill none) (layer "Edge.Cuts"))
 (gr_line (start 134.707462 124.242286) (end 129.757714 119.292538) (stroke (width 0.05) (type default)) (layer "Edge.Cuts"))
 (gr_arc (start 175.042286 83.907462) (mid 175.203432 84.14861) (end 175.26 84.43307) (stroke (width 0.05) (type default))
  (layer "Edge.Cuts"))
 (segment (start 160.025 93.98) (end 165.1 93.98) (width 0.2) (layer "F.Cu") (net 2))
 (segment (start 160.025 96.52) (end 165.1 96.52) (width 0.2) (layer "F.Cu") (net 1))
 (segment (start 139.7 96.52) (end 144.775 96.52) (width 0.2) (layer "F.Cu") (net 4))
 (segment (start 137.16 96.52) (end 139.7 96.52) (width 0.2) (layer "F.Cu") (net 4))
 (segment (start 137.16 93.98) (end 139.7 93.98) (width 0.2) (layer "F.Cu") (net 3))
 (segment (start 139.7 93.98) (end 144.775 93.98) (width 0.2) (layer "F.Cu") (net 3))
 (segment (start 139.67 101.57) (end 139.7 101.6) (width 0.2) (layer "F.Cu") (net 6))
 (segment (start 144.745 101.57) (end 144.775 101.6) (width 0.2) (layer "F.Cu") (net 6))
 (segment (start 137.16 101.57) (end 139.67 101.57) (width 0.2) (layer "F.Cu") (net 6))
 (segment (start 139.7 101.6) (end 144.775 101.6) (width 0.2) (layer "F.Cu") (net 6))
 (segment (start 139.7 99.06) (end 144.775 99.06) (width 0.2) (layer "F.Cu") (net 5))
 (segment (start 137.16 99.06) (end 139.7 99.06) (width 0.2) (layer "F.Cu") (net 5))
 (segment (start 139.7 104.14) (end 144.775 104.14) (width 0.2) (layer "F.Cu") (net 7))
 (segment (start 137.16 104.14) (end 139.7 104.14) (width 0.2) (layer "F.Cu") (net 7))
 (segment (start 137.16 106.68) (end 139.7 106.68) (width 0.2) (layer "F.Cu") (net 8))
 (segment (start 139.7 106.68) (end 144.775 106.68) (width 0.2) (layer "F.Cu") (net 8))
 (segment (start 160.025 101.6) (end 165.1 101.6) (width 0.2) (layer "F.Cu") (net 17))
 (segment (start 160.025 104.14) (end 165.1 104.14) (width 0.2) (layer "F.Cu") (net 16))
 (segment (start 160.025 106.68) (end 165.1 106.68) (width 0.2) (layer "F.Cu") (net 15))
 (segment (start 160.025 99.06) (end 165.1 99.06) (width 0.2) (layer "F.Cu") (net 18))
 (segment (start 160.025 109.22) (end 165.1 109.22) (width 0.2) (layer "F.Cu") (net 14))
 (segment (start 139.7 109.22) (end 144.775 109.22) (width 0.2) (layer "F.Cu") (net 13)))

